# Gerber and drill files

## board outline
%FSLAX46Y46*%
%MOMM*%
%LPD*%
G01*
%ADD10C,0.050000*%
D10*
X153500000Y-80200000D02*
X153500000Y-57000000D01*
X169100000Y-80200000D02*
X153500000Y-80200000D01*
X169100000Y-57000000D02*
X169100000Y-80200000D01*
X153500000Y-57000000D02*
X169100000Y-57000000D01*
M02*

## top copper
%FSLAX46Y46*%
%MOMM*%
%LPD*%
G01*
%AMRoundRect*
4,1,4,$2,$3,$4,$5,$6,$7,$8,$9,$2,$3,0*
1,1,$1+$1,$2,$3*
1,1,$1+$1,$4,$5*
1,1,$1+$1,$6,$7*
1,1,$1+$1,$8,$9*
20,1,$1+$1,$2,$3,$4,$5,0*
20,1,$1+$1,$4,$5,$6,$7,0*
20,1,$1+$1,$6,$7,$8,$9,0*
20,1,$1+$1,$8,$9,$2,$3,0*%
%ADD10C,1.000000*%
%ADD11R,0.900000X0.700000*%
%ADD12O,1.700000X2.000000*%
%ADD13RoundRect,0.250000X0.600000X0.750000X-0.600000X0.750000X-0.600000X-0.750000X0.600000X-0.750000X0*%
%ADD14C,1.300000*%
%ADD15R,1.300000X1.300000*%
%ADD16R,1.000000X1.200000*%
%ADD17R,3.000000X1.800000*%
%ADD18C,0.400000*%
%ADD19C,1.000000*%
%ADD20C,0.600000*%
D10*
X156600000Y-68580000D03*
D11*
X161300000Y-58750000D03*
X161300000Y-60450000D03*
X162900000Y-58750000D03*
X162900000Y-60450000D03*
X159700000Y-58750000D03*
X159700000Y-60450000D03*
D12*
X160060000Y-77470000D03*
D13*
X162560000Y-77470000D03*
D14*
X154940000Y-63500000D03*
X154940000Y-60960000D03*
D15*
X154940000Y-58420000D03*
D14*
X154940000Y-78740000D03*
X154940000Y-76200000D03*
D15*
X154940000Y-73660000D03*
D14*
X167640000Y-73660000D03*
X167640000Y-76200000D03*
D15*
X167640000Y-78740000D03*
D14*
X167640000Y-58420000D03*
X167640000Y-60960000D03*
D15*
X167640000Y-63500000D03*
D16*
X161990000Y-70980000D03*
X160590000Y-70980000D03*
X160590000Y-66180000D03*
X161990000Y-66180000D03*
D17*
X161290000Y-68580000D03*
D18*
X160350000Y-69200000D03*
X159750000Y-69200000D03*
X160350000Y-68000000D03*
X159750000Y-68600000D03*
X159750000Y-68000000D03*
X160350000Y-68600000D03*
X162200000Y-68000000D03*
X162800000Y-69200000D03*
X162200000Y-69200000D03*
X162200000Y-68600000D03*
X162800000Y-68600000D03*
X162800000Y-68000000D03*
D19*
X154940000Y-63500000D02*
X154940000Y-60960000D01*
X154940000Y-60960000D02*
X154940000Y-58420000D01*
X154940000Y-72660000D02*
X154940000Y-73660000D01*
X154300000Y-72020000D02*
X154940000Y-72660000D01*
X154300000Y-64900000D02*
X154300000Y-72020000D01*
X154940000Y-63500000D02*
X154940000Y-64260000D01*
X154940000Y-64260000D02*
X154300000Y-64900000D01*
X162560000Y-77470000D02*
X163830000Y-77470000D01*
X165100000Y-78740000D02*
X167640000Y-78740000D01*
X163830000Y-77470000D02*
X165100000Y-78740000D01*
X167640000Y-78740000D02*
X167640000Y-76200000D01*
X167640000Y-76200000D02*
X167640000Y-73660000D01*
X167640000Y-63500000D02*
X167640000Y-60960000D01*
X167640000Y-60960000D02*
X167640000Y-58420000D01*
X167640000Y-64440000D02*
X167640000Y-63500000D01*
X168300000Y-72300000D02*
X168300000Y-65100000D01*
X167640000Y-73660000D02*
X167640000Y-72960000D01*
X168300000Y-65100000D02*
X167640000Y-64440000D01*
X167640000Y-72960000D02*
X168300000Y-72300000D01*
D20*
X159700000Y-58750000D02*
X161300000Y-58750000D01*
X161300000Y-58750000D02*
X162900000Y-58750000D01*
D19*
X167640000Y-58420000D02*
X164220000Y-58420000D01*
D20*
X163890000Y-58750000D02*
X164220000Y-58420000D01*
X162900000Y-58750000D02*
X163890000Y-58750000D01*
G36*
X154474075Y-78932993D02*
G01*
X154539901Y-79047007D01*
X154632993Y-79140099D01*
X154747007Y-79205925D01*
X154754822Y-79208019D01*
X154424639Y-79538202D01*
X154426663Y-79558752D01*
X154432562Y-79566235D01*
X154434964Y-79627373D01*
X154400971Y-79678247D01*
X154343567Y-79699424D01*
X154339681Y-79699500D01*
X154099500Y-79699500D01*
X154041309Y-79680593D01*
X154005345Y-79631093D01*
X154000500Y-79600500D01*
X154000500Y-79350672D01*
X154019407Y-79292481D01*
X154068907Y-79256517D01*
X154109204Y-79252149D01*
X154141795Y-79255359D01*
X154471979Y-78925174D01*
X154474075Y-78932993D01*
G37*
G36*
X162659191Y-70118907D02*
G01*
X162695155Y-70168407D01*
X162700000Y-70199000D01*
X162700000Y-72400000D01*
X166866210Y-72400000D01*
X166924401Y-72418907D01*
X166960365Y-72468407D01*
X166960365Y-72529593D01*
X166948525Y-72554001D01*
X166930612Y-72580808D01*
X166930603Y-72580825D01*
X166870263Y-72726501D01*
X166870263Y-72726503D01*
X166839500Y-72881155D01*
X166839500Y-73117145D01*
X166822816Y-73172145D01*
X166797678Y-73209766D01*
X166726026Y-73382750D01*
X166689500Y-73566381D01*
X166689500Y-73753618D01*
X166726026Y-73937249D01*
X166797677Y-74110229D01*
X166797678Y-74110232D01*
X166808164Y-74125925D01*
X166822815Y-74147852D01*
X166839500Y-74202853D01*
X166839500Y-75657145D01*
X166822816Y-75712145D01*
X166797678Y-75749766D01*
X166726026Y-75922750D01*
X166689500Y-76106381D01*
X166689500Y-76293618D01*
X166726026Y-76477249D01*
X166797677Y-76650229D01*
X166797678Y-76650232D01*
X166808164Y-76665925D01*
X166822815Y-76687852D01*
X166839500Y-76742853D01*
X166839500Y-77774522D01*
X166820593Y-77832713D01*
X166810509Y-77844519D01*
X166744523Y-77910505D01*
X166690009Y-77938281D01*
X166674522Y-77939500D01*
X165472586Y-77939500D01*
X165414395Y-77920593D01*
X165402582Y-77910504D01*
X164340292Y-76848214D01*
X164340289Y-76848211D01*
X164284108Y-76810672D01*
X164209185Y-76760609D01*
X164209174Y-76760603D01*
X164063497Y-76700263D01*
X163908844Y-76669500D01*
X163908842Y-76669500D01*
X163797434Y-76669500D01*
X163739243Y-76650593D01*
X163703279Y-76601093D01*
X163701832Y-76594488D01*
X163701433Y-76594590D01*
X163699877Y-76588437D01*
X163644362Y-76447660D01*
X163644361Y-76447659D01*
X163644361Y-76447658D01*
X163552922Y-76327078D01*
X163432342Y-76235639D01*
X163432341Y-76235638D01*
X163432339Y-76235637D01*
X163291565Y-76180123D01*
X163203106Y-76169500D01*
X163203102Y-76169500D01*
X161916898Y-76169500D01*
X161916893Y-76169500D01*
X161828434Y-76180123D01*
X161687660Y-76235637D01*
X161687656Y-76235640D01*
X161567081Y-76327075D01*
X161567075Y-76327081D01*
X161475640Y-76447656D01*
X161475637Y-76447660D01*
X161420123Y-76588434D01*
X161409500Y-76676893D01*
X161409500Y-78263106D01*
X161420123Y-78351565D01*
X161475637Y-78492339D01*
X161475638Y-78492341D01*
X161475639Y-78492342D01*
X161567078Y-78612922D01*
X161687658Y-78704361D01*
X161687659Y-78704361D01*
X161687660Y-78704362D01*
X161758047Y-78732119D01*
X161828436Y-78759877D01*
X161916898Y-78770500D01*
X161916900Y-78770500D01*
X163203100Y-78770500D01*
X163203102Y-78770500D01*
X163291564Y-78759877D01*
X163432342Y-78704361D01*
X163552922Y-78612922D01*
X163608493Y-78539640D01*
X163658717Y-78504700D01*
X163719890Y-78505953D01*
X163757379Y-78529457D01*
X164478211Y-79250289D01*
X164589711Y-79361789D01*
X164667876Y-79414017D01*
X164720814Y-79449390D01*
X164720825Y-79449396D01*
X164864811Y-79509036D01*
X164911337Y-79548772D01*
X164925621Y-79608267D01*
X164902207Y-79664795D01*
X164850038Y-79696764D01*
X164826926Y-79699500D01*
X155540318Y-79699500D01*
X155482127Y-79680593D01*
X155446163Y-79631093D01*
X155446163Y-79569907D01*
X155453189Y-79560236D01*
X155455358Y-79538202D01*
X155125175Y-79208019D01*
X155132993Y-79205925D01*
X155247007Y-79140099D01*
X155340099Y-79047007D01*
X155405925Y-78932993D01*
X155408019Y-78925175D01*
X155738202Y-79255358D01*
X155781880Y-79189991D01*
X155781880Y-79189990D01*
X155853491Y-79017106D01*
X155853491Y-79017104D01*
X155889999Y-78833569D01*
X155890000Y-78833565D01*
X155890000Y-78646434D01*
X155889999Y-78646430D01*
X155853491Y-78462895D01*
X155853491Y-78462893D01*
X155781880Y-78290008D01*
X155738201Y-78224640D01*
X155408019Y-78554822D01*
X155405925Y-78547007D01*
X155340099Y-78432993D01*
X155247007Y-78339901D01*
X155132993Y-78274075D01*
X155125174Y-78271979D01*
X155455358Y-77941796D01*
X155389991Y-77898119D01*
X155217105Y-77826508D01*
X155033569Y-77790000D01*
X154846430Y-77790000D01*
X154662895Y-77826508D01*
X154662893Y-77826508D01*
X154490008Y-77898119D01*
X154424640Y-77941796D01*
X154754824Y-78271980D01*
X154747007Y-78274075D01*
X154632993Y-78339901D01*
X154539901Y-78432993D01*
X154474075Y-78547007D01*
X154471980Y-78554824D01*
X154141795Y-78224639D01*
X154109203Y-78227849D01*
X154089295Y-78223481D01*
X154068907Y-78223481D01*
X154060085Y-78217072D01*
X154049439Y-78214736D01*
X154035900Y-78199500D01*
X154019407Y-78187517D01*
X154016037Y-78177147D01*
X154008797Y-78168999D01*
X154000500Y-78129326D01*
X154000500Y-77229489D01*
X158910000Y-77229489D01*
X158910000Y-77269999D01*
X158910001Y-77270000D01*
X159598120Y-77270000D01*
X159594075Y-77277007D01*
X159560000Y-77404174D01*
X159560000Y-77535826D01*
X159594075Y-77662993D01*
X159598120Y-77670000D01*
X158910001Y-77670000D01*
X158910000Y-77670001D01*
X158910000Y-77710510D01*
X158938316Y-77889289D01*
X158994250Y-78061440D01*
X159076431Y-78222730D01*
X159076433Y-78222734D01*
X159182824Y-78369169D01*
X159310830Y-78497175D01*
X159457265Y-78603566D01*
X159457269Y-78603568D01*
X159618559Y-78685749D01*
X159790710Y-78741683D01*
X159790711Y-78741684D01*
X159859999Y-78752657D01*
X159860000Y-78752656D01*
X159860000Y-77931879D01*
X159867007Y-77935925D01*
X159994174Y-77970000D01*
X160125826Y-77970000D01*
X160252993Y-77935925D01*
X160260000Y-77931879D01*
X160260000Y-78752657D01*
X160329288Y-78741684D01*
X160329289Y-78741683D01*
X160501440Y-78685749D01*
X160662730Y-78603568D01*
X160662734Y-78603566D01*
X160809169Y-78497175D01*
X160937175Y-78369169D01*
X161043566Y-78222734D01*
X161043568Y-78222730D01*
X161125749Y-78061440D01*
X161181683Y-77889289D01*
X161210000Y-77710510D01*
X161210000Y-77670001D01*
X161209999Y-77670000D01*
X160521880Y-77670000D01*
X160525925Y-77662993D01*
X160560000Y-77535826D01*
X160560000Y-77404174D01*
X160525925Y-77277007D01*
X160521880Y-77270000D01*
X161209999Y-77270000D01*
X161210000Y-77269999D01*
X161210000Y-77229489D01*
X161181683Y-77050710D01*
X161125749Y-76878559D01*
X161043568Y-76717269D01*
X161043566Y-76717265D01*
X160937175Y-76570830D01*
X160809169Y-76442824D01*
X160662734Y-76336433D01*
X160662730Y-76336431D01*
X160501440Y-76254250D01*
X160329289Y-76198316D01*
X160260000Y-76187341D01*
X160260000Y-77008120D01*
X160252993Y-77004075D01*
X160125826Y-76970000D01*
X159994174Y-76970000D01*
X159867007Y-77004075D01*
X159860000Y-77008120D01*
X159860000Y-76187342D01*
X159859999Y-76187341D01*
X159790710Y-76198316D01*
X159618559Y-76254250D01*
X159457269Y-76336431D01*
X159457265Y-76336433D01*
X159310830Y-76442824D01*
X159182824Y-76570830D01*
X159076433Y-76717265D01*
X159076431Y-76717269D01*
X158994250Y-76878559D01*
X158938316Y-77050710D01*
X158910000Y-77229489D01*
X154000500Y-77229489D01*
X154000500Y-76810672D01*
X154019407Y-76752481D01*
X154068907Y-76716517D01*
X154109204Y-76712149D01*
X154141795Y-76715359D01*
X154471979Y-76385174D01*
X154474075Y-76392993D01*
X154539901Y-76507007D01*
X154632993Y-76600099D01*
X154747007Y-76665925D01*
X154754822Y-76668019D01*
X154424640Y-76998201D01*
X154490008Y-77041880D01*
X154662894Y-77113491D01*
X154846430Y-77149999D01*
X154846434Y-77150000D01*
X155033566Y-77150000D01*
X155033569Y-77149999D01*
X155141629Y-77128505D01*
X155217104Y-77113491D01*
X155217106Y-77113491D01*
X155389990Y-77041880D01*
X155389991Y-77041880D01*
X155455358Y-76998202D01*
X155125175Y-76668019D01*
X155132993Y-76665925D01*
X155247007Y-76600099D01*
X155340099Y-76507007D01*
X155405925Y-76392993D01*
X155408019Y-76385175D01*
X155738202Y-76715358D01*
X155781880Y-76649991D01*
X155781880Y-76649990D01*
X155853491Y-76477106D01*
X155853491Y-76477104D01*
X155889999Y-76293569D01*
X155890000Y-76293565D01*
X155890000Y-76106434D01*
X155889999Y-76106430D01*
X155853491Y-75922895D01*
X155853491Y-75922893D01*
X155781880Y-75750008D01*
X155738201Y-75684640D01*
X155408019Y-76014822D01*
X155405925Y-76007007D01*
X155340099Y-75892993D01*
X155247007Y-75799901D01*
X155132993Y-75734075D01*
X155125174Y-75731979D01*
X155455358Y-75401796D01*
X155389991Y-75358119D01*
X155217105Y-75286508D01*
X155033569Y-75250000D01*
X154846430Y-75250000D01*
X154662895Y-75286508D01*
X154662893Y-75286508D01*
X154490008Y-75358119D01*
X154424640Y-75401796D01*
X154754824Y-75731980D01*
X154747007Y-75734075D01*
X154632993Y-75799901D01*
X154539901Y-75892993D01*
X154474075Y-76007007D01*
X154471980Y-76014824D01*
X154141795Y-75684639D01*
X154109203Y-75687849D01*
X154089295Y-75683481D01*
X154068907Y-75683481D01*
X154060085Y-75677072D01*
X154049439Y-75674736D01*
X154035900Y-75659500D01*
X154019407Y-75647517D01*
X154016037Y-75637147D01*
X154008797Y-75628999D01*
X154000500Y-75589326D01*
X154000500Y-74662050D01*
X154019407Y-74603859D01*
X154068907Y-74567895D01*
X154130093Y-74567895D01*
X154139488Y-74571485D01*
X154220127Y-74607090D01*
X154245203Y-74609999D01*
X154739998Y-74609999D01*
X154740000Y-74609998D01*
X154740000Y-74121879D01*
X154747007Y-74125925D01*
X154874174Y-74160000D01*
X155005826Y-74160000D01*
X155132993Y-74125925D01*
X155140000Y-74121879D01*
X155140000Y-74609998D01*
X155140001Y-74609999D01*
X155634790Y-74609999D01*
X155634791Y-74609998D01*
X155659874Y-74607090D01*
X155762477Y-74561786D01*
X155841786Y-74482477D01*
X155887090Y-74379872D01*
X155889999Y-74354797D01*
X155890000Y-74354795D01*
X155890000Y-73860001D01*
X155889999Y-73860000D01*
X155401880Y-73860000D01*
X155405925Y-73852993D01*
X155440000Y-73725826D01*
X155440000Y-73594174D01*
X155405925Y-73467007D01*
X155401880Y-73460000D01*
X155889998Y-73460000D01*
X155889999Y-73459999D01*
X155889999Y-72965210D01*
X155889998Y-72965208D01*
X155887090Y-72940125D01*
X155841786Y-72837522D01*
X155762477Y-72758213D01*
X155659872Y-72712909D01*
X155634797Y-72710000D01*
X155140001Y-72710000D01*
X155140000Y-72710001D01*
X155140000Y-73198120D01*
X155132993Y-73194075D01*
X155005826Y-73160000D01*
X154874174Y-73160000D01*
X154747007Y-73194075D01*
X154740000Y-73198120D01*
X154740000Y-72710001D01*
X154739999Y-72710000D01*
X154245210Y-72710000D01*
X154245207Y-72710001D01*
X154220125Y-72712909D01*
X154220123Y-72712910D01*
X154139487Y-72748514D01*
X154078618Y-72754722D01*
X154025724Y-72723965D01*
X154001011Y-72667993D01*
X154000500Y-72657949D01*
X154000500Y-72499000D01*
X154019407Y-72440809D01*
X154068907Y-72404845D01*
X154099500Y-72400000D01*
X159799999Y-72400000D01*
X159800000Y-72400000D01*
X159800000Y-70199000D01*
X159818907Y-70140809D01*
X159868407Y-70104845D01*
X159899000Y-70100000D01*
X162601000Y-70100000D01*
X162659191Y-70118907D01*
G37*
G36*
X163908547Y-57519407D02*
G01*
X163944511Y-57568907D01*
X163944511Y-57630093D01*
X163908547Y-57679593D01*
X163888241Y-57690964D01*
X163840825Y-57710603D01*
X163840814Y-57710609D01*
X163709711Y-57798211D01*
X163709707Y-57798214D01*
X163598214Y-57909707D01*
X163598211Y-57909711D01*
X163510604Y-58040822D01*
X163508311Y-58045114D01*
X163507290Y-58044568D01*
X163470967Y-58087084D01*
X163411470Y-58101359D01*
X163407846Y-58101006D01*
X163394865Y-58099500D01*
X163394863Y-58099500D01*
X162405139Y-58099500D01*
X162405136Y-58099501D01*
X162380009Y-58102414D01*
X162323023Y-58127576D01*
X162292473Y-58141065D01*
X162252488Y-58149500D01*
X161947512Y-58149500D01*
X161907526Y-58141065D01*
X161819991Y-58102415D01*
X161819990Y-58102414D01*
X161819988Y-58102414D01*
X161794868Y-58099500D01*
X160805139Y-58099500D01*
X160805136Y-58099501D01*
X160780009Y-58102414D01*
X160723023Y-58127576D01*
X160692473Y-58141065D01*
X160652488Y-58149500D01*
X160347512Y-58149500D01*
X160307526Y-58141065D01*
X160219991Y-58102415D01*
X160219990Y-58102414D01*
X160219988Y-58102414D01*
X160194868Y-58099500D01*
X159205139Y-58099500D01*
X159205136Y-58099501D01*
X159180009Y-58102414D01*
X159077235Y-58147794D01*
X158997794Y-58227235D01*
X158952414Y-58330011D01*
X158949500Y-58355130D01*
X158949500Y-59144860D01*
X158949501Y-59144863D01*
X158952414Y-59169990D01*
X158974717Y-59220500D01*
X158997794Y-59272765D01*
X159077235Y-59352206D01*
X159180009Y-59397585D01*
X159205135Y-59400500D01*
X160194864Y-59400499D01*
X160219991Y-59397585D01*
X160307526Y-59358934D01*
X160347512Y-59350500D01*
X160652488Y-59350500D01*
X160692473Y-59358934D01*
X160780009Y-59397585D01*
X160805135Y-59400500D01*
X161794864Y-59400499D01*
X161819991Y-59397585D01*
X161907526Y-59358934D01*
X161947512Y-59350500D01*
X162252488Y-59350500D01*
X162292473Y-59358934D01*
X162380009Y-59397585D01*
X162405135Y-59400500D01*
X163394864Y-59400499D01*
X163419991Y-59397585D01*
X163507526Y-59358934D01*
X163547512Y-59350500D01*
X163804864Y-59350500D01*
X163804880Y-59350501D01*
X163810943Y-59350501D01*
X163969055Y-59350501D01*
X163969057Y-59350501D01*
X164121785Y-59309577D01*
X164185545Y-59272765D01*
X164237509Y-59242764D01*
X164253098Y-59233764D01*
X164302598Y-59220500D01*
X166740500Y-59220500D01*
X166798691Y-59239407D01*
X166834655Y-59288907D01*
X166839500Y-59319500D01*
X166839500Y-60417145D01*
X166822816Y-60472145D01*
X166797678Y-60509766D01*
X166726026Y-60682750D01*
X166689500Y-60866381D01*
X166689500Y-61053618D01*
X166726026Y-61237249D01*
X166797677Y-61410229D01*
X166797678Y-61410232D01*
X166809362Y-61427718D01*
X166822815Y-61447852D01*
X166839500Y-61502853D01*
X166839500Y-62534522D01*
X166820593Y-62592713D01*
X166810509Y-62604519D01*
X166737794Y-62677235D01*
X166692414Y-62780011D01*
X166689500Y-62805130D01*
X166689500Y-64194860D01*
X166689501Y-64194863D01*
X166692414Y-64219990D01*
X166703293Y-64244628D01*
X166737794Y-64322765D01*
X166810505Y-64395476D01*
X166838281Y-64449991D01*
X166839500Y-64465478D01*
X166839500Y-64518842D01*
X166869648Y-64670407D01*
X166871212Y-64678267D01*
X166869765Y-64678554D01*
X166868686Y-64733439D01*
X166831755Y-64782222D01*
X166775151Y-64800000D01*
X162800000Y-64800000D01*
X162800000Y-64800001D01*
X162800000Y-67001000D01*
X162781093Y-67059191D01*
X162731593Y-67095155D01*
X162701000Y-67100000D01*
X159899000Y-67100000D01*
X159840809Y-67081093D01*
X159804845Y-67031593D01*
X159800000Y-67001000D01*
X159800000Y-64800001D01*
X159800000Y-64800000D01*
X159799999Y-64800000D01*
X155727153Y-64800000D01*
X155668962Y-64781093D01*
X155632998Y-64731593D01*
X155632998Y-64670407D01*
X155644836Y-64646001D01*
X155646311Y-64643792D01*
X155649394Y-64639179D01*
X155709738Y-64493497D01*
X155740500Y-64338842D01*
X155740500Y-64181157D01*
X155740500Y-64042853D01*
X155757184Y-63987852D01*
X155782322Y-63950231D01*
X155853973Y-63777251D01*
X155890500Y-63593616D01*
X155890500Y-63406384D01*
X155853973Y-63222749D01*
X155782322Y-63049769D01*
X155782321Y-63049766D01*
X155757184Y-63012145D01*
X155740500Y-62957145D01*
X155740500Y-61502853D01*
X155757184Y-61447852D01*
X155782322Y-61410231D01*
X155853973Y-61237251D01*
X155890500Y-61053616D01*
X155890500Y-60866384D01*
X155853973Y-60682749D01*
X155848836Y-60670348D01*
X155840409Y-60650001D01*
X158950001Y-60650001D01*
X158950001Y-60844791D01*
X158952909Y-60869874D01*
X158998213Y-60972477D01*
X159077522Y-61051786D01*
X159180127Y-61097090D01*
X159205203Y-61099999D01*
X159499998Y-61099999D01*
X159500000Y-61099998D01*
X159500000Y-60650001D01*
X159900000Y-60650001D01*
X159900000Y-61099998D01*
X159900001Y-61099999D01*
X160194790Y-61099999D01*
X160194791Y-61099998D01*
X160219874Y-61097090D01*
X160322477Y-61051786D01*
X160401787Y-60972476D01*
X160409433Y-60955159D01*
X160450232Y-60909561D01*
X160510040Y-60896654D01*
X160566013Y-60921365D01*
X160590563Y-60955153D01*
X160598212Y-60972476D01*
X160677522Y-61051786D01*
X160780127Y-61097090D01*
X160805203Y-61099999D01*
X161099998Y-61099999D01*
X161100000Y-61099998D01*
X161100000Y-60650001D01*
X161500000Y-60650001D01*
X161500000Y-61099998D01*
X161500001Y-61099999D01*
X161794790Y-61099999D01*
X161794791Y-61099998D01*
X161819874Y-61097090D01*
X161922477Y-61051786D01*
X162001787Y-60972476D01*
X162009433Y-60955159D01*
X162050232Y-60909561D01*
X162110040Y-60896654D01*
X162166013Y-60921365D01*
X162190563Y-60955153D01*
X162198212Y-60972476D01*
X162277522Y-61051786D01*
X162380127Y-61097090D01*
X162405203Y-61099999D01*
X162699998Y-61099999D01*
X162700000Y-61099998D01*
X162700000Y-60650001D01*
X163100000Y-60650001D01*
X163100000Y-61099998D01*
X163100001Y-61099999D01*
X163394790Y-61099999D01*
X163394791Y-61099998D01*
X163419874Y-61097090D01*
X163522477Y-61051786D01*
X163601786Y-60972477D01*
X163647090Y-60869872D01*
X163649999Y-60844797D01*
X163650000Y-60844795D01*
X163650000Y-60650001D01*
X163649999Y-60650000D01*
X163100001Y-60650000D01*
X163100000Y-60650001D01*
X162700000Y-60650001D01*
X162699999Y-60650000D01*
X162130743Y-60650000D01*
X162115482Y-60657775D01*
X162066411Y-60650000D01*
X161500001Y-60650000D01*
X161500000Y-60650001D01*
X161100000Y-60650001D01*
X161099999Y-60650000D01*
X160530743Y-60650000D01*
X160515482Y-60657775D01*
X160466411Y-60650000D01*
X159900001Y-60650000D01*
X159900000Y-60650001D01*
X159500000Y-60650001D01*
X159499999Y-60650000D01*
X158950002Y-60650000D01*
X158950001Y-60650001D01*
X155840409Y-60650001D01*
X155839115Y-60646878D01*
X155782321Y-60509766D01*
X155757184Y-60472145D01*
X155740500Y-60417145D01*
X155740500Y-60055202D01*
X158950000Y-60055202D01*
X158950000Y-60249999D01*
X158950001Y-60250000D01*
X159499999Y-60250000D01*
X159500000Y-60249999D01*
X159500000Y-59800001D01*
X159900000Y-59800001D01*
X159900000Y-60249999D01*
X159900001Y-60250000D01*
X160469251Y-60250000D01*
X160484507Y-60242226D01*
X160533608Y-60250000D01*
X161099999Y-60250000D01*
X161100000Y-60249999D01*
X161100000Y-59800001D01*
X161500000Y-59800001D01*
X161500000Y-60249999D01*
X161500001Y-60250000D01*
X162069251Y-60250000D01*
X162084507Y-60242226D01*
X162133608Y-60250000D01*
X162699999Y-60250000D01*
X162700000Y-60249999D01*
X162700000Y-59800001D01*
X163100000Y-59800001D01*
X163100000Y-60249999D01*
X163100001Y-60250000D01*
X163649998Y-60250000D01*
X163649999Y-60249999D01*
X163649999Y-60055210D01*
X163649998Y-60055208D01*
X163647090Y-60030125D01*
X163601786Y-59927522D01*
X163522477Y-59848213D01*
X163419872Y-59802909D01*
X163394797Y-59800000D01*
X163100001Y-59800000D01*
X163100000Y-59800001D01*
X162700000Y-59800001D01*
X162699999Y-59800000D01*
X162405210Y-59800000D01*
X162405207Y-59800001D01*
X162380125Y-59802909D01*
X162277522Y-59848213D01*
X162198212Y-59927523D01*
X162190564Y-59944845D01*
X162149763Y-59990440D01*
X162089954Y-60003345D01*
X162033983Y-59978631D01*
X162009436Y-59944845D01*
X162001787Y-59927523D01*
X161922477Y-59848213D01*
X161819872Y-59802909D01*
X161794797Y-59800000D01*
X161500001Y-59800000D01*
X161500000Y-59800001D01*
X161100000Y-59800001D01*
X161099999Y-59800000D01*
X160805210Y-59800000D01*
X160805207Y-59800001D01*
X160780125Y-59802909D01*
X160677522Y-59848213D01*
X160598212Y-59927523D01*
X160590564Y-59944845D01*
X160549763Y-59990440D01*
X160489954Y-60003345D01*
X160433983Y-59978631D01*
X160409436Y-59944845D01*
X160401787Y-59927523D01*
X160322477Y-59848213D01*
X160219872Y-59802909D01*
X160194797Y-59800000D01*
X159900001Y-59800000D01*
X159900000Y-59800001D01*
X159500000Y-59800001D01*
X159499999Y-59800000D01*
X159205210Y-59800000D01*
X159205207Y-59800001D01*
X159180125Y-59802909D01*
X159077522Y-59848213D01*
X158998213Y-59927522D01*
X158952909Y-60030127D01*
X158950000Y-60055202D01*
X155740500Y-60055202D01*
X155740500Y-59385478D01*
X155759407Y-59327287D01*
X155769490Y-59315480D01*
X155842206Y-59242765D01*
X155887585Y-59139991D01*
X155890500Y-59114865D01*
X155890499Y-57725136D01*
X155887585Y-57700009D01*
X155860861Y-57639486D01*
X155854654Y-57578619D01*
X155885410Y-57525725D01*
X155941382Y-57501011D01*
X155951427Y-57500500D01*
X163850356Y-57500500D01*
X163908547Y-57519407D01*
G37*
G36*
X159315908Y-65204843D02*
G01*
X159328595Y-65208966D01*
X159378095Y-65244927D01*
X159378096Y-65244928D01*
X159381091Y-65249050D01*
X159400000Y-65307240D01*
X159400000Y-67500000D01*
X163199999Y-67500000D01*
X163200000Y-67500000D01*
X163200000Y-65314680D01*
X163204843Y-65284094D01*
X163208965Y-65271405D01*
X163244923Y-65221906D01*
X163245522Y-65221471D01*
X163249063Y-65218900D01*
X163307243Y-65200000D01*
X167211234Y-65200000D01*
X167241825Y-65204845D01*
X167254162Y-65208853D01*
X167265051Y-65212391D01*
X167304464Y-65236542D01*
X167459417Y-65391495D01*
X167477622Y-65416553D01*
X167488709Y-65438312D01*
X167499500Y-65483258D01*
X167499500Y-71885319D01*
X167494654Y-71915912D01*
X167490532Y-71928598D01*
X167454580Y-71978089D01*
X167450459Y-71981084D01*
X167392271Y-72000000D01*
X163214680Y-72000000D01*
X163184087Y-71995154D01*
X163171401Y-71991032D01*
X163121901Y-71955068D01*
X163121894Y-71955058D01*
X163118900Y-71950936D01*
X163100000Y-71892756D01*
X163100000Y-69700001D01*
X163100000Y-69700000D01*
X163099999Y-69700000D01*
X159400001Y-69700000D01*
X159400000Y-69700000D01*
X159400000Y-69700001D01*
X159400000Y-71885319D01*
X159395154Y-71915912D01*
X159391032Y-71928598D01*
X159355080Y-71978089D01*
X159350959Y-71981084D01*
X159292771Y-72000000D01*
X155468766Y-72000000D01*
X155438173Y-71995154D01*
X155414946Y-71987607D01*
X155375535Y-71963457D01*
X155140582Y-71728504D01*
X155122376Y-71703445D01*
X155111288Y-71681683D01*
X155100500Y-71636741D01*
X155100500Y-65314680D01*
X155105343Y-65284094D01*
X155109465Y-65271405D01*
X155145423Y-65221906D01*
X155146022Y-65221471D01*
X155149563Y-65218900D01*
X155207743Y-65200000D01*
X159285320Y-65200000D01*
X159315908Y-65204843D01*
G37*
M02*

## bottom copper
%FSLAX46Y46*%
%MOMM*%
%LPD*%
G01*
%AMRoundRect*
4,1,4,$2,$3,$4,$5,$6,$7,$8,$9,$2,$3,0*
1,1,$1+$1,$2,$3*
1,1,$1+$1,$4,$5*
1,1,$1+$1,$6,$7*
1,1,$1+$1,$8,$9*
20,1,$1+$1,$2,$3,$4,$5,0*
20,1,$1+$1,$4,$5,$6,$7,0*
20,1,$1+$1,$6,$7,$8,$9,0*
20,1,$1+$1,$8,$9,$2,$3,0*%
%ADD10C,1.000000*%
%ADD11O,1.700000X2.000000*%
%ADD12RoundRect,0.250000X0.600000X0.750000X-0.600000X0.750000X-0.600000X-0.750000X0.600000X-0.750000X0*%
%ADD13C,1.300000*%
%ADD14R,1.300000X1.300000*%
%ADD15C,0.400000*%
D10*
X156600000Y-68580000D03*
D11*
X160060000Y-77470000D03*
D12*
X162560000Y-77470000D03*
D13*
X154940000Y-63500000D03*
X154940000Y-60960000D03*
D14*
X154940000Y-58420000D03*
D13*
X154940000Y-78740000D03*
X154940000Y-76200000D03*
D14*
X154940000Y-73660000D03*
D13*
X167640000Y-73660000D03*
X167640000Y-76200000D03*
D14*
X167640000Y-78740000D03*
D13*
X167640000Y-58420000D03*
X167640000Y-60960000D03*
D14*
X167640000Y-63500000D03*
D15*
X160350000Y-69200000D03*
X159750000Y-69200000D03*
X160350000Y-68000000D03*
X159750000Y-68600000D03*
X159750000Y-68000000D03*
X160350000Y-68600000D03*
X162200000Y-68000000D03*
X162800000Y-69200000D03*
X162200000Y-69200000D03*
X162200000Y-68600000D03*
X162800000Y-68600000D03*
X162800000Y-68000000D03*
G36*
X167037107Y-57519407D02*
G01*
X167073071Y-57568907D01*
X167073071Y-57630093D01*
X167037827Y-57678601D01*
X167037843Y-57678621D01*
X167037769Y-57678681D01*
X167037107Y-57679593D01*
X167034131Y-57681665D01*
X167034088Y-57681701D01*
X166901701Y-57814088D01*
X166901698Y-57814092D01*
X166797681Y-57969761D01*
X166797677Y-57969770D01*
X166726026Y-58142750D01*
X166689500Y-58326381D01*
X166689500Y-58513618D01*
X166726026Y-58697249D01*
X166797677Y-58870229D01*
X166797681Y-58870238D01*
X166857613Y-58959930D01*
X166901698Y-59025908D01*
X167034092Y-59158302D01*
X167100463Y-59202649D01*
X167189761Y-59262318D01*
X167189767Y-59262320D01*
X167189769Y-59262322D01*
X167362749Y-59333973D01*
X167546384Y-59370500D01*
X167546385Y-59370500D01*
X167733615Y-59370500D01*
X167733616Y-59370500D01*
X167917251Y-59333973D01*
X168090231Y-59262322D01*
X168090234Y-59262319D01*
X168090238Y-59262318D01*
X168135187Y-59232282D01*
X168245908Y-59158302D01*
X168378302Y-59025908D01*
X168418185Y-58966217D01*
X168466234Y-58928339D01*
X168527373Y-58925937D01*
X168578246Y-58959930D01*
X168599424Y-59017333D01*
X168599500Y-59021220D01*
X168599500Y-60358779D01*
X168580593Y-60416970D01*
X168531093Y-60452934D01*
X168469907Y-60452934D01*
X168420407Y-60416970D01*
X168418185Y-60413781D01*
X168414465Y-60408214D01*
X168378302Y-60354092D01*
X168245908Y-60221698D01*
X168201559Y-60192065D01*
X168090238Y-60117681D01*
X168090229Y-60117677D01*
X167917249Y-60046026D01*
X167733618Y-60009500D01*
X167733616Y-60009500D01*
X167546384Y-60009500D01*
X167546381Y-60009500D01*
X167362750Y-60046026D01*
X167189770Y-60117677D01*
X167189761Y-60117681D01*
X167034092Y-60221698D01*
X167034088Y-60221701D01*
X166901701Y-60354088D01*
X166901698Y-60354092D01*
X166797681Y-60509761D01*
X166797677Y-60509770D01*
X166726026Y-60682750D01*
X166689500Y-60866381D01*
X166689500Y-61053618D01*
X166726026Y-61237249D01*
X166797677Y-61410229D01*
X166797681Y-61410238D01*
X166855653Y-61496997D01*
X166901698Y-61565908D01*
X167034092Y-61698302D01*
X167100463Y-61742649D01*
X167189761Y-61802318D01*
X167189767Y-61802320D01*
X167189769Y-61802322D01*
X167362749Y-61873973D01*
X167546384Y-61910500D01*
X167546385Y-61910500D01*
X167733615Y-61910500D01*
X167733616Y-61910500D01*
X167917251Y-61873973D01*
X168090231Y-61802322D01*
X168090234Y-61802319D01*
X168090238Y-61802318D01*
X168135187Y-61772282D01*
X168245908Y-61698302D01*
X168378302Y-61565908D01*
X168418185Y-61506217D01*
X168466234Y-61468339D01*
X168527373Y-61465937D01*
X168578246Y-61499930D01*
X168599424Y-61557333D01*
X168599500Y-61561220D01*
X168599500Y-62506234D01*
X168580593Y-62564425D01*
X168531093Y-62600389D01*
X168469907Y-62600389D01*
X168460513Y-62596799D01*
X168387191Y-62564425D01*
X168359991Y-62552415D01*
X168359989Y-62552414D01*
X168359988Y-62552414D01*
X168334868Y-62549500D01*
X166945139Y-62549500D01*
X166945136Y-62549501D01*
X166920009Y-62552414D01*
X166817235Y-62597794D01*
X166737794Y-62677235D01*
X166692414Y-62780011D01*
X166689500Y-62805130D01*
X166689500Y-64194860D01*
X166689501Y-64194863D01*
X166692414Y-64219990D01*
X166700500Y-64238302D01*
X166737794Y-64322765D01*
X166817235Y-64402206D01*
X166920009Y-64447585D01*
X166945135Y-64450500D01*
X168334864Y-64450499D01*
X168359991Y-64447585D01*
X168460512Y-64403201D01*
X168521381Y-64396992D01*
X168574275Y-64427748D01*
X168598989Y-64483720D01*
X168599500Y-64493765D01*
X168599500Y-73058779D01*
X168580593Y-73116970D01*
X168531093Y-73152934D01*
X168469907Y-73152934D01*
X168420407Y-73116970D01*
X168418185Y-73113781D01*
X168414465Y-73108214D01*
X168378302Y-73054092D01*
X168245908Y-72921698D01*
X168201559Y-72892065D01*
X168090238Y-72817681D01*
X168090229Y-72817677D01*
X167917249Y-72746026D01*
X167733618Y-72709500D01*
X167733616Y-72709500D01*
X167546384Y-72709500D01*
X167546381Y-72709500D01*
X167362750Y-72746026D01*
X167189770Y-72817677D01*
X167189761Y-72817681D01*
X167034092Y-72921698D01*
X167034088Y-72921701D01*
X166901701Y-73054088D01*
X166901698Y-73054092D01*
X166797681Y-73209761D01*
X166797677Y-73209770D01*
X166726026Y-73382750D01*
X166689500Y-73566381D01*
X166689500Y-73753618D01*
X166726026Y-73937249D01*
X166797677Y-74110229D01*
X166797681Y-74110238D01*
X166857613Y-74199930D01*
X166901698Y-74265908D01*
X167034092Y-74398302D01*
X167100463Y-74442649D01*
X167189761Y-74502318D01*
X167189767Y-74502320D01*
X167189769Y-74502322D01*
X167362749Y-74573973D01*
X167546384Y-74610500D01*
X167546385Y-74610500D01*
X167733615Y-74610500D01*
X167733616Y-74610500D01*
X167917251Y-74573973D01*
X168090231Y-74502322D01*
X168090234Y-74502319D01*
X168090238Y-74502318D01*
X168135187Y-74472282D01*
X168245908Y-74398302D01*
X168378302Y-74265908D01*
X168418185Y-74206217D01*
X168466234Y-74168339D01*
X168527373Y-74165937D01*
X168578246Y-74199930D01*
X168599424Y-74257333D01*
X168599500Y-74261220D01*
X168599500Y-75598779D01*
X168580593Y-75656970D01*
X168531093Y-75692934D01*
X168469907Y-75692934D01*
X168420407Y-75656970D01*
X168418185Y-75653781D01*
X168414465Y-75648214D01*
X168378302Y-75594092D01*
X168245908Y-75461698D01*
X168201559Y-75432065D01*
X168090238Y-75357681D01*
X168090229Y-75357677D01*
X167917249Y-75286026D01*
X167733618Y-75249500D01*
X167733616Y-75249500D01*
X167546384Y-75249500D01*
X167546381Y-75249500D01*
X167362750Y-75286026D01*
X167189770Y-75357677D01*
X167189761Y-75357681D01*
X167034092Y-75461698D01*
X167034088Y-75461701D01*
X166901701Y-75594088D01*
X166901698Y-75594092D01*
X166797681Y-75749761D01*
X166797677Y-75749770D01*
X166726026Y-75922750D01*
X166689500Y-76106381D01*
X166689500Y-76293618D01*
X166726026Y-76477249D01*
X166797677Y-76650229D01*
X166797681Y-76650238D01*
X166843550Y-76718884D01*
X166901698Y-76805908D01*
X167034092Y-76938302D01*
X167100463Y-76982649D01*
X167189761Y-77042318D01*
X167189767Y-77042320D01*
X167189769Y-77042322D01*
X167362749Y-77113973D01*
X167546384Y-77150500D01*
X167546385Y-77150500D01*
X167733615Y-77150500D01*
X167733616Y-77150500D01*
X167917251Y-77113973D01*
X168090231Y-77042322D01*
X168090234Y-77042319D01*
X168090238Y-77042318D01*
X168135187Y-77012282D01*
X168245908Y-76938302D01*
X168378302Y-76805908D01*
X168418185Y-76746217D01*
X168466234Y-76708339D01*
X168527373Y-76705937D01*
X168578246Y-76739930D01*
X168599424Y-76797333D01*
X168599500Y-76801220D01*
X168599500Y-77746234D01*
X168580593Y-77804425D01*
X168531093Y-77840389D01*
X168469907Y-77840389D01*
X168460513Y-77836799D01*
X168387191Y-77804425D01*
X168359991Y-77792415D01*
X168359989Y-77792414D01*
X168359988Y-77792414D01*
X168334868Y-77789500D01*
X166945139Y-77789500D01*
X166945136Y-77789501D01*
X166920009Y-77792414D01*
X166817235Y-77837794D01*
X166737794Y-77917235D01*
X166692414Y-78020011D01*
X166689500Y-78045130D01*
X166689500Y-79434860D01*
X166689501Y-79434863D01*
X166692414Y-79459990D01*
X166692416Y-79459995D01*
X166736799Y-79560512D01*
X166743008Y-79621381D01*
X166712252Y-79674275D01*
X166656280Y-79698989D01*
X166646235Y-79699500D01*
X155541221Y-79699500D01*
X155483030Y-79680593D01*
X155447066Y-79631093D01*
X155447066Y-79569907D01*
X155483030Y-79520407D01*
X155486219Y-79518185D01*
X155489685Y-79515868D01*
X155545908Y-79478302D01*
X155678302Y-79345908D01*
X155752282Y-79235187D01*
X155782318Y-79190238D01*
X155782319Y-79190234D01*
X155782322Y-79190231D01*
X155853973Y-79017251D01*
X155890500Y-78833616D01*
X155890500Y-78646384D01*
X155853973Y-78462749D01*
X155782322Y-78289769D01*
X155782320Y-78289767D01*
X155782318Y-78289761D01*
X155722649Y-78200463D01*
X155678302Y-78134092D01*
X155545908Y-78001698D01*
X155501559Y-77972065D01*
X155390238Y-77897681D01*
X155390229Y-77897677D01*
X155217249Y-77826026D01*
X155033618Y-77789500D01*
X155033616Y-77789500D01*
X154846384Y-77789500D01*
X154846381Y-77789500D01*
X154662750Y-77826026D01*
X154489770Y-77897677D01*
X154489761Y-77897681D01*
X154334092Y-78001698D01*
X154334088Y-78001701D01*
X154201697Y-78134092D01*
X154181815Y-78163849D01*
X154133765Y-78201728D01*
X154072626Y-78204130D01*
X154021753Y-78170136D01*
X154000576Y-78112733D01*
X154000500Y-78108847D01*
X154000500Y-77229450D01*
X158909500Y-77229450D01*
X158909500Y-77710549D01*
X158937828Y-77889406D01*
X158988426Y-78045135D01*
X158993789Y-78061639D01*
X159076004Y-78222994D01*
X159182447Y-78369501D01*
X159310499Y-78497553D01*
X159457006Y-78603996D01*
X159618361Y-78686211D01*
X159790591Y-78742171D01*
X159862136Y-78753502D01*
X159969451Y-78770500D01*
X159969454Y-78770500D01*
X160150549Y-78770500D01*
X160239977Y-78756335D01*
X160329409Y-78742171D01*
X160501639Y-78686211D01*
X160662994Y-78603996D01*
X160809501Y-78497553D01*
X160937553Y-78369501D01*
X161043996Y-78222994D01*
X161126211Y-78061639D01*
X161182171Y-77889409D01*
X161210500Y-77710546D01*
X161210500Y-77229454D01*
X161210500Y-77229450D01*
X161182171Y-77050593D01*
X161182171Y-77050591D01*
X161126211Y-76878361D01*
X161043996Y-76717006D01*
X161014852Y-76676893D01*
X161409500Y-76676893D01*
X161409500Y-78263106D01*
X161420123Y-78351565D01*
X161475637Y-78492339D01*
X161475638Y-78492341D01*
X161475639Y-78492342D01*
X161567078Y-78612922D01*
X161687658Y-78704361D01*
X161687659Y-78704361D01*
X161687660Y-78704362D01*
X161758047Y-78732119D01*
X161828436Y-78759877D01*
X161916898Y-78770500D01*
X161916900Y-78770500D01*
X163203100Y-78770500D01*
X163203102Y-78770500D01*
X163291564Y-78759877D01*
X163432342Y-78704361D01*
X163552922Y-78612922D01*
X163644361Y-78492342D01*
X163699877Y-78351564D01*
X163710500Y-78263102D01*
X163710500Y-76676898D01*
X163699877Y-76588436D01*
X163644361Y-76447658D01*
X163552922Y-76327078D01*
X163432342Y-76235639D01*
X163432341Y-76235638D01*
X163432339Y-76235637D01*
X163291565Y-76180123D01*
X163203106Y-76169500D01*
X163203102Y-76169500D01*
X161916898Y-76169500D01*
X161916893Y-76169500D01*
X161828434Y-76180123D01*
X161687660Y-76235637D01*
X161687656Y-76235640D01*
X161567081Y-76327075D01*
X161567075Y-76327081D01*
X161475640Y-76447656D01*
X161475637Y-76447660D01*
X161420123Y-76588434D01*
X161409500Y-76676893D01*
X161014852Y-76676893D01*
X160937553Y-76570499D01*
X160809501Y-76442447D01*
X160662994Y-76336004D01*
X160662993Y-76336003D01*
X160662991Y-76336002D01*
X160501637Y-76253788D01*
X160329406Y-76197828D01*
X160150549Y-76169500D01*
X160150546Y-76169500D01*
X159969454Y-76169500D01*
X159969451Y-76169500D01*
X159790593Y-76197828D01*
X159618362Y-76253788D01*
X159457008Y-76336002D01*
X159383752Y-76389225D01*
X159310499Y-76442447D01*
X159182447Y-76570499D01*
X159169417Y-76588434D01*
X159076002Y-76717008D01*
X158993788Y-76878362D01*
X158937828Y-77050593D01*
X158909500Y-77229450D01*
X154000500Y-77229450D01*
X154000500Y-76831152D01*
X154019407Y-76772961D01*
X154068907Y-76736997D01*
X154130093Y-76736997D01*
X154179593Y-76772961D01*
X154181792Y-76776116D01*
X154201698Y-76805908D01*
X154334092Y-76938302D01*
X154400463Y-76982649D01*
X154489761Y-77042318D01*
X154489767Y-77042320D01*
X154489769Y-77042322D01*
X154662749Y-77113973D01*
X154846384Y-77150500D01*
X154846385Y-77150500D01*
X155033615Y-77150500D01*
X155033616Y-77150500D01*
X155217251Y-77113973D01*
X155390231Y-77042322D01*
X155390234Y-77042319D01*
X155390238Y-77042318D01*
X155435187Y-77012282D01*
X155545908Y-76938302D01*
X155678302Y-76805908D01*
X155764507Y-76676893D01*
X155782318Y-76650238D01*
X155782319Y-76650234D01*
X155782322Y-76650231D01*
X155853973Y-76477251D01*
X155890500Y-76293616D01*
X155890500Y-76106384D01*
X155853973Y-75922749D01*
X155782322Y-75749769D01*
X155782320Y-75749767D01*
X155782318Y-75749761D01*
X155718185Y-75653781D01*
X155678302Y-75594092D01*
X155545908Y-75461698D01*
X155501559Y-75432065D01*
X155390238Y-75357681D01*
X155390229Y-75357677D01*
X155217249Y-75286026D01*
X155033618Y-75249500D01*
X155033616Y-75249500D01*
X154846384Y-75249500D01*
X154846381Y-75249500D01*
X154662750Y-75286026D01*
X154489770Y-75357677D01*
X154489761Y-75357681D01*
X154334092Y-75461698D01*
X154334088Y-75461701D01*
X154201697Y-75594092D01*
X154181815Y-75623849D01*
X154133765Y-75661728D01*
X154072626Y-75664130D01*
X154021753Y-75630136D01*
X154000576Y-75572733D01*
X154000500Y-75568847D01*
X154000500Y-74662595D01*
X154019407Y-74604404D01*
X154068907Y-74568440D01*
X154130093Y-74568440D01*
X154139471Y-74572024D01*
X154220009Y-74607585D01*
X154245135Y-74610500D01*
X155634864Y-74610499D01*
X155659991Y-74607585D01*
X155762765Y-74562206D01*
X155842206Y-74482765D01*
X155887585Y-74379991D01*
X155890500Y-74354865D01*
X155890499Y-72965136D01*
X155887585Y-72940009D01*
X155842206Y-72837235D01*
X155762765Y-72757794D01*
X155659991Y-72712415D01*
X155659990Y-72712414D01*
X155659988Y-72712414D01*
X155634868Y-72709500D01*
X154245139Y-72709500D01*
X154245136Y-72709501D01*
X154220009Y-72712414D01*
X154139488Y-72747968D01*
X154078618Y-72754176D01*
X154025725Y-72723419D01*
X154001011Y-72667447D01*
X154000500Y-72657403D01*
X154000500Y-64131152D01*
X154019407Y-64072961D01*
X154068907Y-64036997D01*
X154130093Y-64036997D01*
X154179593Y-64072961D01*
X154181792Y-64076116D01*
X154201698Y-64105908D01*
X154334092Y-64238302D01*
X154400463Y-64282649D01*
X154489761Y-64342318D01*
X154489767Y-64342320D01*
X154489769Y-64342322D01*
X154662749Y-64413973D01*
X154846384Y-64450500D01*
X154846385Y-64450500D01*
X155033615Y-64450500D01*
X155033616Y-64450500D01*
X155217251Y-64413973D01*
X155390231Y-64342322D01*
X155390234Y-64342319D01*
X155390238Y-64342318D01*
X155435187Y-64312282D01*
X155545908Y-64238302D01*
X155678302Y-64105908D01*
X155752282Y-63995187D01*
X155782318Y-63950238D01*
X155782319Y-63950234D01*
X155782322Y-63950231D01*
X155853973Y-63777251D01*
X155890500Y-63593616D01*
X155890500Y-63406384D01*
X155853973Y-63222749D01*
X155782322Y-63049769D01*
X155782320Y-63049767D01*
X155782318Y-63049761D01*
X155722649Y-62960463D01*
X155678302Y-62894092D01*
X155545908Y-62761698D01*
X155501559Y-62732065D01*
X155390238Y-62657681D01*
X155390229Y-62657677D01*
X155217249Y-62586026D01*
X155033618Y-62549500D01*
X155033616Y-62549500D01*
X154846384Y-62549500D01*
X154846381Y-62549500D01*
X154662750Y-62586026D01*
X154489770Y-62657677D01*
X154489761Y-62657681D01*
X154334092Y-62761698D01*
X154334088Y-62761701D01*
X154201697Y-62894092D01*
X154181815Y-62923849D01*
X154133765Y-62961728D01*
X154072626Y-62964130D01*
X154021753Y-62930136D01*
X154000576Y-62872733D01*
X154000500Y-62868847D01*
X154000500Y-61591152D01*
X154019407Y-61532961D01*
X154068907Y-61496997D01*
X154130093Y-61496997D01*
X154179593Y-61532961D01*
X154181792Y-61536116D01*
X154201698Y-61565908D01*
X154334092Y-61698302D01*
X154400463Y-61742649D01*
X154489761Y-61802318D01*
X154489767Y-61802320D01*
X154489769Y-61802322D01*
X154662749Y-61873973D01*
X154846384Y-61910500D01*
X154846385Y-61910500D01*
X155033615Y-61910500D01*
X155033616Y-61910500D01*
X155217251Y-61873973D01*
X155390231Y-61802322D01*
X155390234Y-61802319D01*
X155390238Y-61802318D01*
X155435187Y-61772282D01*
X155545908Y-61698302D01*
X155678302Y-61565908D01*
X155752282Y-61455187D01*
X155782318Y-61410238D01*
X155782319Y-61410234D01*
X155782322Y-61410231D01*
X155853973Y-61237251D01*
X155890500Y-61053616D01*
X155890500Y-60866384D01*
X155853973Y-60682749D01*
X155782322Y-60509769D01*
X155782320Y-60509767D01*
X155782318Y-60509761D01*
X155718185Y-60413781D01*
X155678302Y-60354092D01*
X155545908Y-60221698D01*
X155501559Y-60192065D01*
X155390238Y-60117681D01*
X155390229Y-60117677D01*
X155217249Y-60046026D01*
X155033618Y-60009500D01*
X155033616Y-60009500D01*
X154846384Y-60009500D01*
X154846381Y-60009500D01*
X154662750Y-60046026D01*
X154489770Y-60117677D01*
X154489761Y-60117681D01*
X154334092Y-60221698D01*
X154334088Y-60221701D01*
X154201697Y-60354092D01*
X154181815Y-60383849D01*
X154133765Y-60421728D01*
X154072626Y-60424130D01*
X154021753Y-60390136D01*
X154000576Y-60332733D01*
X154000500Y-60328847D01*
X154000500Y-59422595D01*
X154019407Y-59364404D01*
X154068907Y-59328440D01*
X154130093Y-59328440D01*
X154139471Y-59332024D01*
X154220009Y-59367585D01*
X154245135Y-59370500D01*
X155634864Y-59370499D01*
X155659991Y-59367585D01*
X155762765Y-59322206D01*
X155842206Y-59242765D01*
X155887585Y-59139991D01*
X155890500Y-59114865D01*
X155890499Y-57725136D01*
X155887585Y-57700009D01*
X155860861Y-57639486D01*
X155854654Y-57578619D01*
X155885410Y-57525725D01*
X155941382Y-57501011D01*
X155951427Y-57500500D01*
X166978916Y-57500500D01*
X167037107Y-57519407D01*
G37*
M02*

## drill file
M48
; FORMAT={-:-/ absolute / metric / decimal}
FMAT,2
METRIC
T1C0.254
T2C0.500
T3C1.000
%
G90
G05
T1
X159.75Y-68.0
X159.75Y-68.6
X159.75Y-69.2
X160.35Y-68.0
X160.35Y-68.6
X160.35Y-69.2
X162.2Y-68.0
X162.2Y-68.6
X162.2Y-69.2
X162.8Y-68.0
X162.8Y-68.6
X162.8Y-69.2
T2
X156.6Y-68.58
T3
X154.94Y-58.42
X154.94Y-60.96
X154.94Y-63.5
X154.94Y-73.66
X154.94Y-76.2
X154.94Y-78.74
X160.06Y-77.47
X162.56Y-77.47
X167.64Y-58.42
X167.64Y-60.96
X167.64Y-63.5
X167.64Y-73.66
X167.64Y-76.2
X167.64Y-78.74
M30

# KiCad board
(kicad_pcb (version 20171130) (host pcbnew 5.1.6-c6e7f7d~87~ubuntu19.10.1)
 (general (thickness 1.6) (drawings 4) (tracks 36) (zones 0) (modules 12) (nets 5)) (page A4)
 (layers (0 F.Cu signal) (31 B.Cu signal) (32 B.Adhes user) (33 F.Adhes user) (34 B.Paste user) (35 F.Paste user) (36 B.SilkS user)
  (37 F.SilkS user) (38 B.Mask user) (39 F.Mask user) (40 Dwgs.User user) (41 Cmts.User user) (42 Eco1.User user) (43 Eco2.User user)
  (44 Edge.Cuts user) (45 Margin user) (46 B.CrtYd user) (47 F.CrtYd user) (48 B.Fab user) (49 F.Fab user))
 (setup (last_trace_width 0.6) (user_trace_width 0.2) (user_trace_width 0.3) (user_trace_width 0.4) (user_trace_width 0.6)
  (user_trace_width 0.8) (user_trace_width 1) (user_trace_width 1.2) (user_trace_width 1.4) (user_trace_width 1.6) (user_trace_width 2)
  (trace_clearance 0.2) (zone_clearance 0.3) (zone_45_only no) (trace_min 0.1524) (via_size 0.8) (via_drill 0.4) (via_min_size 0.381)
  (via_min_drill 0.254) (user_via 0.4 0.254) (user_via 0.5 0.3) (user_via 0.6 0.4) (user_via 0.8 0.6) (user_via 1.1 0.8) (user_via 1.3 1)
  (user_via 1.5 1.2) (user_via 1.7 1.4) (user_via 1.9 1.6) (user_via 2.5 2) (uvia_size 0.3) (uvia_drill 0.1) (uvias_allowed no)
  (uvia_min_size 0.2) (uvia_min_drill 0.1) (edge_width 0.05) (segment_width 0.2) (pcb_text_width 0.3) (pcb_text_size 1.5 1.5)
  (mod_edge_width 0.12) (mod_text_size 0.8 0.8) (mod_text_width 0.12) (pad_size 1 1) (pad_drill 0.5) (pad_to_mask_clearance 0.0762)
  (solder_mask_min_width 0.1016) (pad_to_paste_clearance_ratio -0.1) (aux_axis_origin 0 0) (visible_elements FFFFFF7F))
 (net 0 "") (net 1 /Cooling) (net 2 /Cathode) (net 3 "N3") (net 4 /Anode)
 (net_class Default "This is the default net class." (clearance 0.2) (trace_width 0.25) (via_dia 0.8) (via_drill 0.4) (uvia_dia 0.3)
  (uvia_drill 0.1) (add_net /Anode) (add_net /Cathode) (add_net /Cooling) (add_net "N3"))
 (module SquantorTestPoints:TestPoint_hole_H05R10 (layer F.Cu) (at 156.6 68.58)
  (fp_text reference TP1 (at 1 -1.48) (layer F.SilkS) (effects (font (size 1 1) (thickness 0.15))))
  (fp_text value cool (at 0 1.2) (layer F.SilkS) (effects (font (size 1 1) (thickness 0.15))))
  (pad 1 thru_hole circle (at 0 0) (size 1 1) (drill 0.5) (layers *.Cu *.Mask) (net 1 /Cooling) (zone_connect 2)))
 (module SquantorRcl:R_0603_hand (layer F.Cu) (at 161.3 59.6 90)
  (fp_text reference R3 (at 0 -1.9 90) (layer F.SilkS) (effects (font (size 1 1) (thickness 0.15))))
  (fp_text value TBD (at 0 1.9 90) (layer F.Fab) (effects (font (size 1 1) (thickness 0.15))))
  (pad 2 smd rect (at 0.85 0 90) (size 0.7 0.9) (layers F.Cu F.Paste F.Mask) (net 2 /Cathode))
  (pad 1 smd rect (at -0.85 0 90) (size 0.7 0.9) (layers F.Cu F.Paste F.Mask) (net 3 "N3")))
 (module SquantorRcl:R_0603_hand (layer F.Cu) (at 162.9 59.6 90)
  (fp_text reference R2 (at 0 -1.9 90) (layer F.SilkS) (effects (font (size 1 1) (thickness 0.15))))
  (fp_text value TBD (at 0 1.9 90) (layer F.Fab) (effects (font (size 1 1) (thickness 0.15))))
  (pad 2 smd rect (at 0.85 0 90) (size 0.7 0.9) (layers F.Cu F.Paste F.Mask) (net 2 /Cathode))
  (pad 1 smd rect (at -0.85 0 90) (size 0.7 0.9) (layers F.Cu F.Paste F.Mask) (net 3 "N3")))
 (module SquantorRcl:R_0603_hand (layer F.Cu) (at 159.7 59.6 90)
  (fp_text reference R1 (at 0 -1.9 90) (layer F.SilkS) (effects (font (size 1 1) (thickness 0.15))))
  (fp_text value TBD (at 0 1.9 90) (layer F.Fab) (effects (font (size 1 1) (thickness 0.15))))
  (pad 2 smd rect (at 0.85 0 90) (size 0.7 0.9) (layers F.Cu F.Paste F.Mask) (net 2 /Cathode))
  (pad 1 smd rect (at -0.85 0 90) (size 0.7 0.9) (layers F.Cu F.Paste F.Mask) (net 3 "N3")))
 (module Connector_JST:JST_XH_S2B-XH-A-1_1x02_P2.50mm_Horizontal (layer B.Cu) (at 162.56 77.47 180)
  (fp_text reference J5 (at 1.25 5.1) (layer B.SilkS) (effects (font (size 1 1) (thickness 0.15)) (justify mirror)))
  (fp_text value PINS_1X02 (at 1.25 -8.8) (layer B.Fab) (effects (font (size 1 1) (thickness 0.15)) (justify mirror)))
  (pad 2 thru_hole oval (at 2.5 0 180) (size 1.7 2) (drill 1) (layers *.Cu *.Mask) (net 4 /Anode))
  (pad 1 thru_hole roundrect (at 0 0 180) (size 1.7 2) (drill 1) (layers *.Cu *.Mask) (roundrect_rratio 0.147059) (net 2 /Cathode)))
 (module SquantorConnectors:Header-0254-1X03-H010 (layer F.Cu) (at 154.94 60.96 270)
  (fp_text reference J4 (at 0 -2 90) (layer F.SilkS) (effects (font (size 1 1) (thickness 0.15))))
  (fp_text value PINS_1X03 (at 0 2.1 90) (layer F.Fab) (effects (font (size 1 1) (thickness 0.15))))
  (pad 3 thru_hole circle (at 2.54 0 90) (size 1.3 1.3) (drill 1) (layers *.Cu *.Mask) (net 4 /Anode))
  (pad 2 thru_hole circle (at 0 0 90) (size 1.3 1.3) (drill 1) (layers *.Cu *.Mask) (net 4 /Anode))
  (pad 1 thru_hole rect (at -2.54 0 90) (size 1.3 1.3) (drill 1) (layers *.Cu *.Mask) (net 4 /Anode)))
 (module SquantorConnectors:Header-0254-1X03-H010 (layer F.Cu) (at 154.94 76.2 270)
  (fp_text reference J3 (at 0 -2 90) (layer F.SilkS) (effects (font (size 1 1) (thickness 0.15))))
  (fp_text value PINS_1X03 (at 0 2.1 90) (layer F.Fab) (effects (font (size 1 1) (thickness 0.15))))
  (pad 3 thru_hole circle (at 2.54 0 90) (size 1.3 1.3) (drill 1) (layers *.Cu *.Mask) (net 4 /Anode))
  (pad 2 thru_hole circle (at 0 0 90) (size 1.3 1.3) (drill 1) (layers *.Cu *.Mask) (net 4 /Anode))
  (pad 1 thru_hole rect (at -2.54 0 90) (size 1.3 1.3) (drill 1) (layers *.Cu *.Mask) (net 4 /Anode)))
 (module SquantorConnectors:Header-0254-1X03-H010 (layer F.Cu) (at 167.64 76.2 90)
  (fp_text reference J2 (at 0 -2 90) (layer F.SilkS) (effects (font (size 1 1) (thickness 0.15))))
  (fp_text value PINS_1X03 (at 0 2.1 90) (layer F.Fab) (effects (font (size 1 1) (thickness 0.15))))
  (pad 3 thru_hole circle (at 2.54 0 270) (size 1.3 1.3) (drill 1) (layers *.Cu *.Mask) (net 2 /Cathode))
  (pad 2 thru_hole circle (at 0 0 270) (size 1.3 1.3) (drill 1) (layers *.Cu *.Mask) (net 2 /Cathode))
  (pad 1 thru_hole rect (at -2.54 0 270) (size 1.3 1.3) (drill 1) (layers *.Cu *.Mask) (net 2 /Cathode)))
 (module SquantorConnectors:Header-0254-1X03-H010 (layer F.Cu) (at 167.64 60.96 90)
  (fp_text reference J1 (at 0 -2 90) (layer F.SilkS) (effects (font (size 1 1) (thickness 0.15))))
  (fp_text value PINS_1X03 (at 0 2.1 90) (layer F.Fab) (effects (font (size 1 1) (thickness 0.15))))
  (pad 3 thru_hole circle (at 2.54 0 270) (size 1.3 1.3) (drill 1) (layers *.Cu *.Mask) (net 2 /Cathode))
  (pad 2 thru_hole circle (at 0 0 270) (size 1.3 1.3) (drill 1) (layers *.Cu *.Mask) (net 2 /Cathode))
  (pad 1 thru_hole rect (at -2.54 0 270) (size 1.3 1.3) (drill 1) (layers *.Cu *.Mask) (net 2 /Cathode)))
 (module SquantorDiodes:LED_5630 (layer F.Cu) (at 161.29 68.58 270) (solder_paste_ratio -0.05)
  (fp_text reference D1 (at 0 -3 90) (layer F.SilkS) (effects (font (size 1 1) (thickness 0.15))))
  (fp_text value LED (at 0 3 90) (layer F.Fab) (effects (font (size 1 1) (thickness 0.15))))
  (pad 2 smd rect (at 2.4 -0.7 270) (size 1.2 1) (layers F.Cu F.Paste F.Mask) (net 4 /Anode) (zone_connect 2))
  (pad 2 smd rect (at 2.4 0.7 270) (size 1.2 1) (layers F.Cu F.Paste F.Mask) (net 4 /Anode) (zone_connect 2))
  (pad 1 smd rect (at -2.4 0.7 270) (size 1.2 1) (layers F.Cu F.Paste F.Mask) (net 3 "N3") (zone_connect 2))
  (pad 1 smd rect (at -2.4 -0.7 270) (size 1.2 1) (layers F.Cu F.Paste F.Mask) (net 3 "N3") (zone_connect 2))
  (pad 3 smd rect (at 0 0 270) (size 1.8 3) (layers F.Cu) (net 1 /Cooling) (zone_connect 2)))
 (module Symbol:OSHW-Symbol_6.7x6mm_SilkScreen (layer F.Cu) (at 138.7 87.6)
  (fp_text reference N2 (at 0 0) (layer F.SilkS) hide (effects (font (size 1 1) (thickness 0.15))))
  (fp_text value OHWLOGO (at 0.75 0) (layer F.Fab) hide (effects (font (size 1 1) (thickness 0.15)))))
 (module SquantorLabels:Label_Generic (layer F.Cu) (at 138.1 91.5)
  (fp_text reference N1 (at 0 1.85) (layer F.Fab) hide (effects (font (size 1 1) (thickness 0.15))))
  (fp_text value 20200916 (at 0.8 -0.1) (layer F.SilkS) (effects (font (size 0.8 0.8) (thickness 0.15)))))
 (gr_line (start 153.5 80.2) (end 153.5 57) (layer Edge.Cuts) (width 0.05))
 (gr_line (start 169.1 80.2) (end 153.5 80.2) (layer Edge.Cuts) (width 0.05))
 (gr_line (start 169.1 57) (end 169.1 80.2) (layer Edge.Cuts) (width 0.05))
 (gr_line (start 153.5 57) (end 169.1 57) (layer Edge.Cuts) (width 0.05))
 (via (at 160.35 69.2) (size 0.4) (drill 0.254) (layers F.Cu B.Cu) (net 1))
 (via (at 159.75 69.2) (size 0.4) (drill 0.254) (layers F.Cu B.Cu) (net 1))
 (via (at 160.35 68) (size 0.4) (drill 0.254) (layers F.Cu B.Cu) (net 1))
 (via (at 159.75 68.6) (size 0.4) (drill 0.254) (layers F.Cu B.Cu) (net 1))
 (via (at 159.75 68) (size 0.4) (drill 0.254) (layers F.Cu B.Cu) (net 1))
 (segment (start 154.94 63.5) (end 154.94 60.96) (width 1) (layer F.Cu) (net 4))
 (segment (start 154.94 60.96) (end 154.94 58.42) (width 1) (layer F.Cu) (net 4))
 (segment (start 154.94 72.66) (end 154.94 73.66) (width 1) (layer F.Cu) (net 4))
 (segment (start 154.3 72.02) (end 154.94 72.66) (width 1) (layer F.Cu) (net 4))
 (segment (start 154.3 64.9) (end 154.3 72.02) (width 1) (layer F.Cu) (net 4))
 (segment (start 154.94 63.5) (end 154.94 64.26) (width 1) (layer F.Cu) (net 4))
 (segment (start 154.94 64.26) (end 154.3 64.9) (width 1) (layer F.Cu) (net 4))
 (segment (start 162.56 77.47) (end 163.83 77.47) (width 1) (layer F.Cu) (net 2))
 (segment (start 165.1 78.74) (end 167.64 78.74) (width 1) (layer F.Cu) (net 2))
 (segment (start 163.83 77.47) (end 165.1 78.74) (width 1) (layer F.Cu) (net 2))
 (segment (start 167.64 78.74) (end 167.64 76.2) (width 1) (layer F.Cu) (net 2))
 (segment (start 167.64 76.2) (end 167.64 73.66) (width 1) (layer F.Cu) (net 2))
 (segment (start 167.64 63.5) (end 167.64 60.96) (width 1) (layer F.Cu) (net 2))
 (segment (start 167.64 60.96) (end 167.64 58.42) (width 1) (layer F.Cu) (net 2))
 (segment (start 167.64 64.44) (end 167.64 63.5) (width 1) (layer F.Cu) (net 2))
 (segment (start 168.3 72.3) (end 168.3 65.1) (width 1) (layer F.Cu) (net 2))
 (segment (start 167.64 73.66) (end 167.64 72.96) (width 1) (layer F.Cu) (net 2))
 (segment (start 168.3 65.1) (end 167.64 64.44) (width 1) (layer F.Cu) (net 2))
 (segment (start 167.64 72.96) (end 168.3 72.3) (width 1) (layer F.Cu) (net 2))
 (segment (start 159.7 58.75) (end 161.3 58.75) (width 0.6) (layer F.Cu) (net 2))
 (segment (start 161.3 58.75) (end 162.9 58.75) (width 0.6) (layer F.Cu) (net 2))
 (segment (start 167.64 58.42) (end 164.22 58.42) (width 1) (layer F.Cu) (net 2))
 (segment (start 163.89 58.75) (end 164.22 58.42) (width 0.6) (layer F.Cu) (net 2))
 (segment (start 162.9 58.75) (end 163.89 58.75) (width 0.6) (layer F.Cu) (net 2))
 (via (at 160.35 68.6) (size 0.4) (drill 0.254) (layers F.Cu B.Cu) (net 1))
 (via (at 162.2 68) (size 0.4) (drill 0.254) (layers F.Cu B.Cu) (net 1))
 (via (at 162.8 69.2) (size 0.4) (drill 0.254) (layers F.Cu B.Cu) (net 1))
 (via (at 162.2 69.2) (size 0.4) (drill 0.254) (layers F.Cu B.Cu) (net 1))
 (via (at 162.2 68.6) (size 0.4) (drill 0.254) (layers F.Cu B.Cu) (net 1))
 (via (at 162.8 68.6) (size 0.4) (drill 0.254) (layers F.Cu B.Cu) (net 1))
 (via (at 162.8 68) (size 0.4) (drill 0.254) (layers F.Cu B.Cu) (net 1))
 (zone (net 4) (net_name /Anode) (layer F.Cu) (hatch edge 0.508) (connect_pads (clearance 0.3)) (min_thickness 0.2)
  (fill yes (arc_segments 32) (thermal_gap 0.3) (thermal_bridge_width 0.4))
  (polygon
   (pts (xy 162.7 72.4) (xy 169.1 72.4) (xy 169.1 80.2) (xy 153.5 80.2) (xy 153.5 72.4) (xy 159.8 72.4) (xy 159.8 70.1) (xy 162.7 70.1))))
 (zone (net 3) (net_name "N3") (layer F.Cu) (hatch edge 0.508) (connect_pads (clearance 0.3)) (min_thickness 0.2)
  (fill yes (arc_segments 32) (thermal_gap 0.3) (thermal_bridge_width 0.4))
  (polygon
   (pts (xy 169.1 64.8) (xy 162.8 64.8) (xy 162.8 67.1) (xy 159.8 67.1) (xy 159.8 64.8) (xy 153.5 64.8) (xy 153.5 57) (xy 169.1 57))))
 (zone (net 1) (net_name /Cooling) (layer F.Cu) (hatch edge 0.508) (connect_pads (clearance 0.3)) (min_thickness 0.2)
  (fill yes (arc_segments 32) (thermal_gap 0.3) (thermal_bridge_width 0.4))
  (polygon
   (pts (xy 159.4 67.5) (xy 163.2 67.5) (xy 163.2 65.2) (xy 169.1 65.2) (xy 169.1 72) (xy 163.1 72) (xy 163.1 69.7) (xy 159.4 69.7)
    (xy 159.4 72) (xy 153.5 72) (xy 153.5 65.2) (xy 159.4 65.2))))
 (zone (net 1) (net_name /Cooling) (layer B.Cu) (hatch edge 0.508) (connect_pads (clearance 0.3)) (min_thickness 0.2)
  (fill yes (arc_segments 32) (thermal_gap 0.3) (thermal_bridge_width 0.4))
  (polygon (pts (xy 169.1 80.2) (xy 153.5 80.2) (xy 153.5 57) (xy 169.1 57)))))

